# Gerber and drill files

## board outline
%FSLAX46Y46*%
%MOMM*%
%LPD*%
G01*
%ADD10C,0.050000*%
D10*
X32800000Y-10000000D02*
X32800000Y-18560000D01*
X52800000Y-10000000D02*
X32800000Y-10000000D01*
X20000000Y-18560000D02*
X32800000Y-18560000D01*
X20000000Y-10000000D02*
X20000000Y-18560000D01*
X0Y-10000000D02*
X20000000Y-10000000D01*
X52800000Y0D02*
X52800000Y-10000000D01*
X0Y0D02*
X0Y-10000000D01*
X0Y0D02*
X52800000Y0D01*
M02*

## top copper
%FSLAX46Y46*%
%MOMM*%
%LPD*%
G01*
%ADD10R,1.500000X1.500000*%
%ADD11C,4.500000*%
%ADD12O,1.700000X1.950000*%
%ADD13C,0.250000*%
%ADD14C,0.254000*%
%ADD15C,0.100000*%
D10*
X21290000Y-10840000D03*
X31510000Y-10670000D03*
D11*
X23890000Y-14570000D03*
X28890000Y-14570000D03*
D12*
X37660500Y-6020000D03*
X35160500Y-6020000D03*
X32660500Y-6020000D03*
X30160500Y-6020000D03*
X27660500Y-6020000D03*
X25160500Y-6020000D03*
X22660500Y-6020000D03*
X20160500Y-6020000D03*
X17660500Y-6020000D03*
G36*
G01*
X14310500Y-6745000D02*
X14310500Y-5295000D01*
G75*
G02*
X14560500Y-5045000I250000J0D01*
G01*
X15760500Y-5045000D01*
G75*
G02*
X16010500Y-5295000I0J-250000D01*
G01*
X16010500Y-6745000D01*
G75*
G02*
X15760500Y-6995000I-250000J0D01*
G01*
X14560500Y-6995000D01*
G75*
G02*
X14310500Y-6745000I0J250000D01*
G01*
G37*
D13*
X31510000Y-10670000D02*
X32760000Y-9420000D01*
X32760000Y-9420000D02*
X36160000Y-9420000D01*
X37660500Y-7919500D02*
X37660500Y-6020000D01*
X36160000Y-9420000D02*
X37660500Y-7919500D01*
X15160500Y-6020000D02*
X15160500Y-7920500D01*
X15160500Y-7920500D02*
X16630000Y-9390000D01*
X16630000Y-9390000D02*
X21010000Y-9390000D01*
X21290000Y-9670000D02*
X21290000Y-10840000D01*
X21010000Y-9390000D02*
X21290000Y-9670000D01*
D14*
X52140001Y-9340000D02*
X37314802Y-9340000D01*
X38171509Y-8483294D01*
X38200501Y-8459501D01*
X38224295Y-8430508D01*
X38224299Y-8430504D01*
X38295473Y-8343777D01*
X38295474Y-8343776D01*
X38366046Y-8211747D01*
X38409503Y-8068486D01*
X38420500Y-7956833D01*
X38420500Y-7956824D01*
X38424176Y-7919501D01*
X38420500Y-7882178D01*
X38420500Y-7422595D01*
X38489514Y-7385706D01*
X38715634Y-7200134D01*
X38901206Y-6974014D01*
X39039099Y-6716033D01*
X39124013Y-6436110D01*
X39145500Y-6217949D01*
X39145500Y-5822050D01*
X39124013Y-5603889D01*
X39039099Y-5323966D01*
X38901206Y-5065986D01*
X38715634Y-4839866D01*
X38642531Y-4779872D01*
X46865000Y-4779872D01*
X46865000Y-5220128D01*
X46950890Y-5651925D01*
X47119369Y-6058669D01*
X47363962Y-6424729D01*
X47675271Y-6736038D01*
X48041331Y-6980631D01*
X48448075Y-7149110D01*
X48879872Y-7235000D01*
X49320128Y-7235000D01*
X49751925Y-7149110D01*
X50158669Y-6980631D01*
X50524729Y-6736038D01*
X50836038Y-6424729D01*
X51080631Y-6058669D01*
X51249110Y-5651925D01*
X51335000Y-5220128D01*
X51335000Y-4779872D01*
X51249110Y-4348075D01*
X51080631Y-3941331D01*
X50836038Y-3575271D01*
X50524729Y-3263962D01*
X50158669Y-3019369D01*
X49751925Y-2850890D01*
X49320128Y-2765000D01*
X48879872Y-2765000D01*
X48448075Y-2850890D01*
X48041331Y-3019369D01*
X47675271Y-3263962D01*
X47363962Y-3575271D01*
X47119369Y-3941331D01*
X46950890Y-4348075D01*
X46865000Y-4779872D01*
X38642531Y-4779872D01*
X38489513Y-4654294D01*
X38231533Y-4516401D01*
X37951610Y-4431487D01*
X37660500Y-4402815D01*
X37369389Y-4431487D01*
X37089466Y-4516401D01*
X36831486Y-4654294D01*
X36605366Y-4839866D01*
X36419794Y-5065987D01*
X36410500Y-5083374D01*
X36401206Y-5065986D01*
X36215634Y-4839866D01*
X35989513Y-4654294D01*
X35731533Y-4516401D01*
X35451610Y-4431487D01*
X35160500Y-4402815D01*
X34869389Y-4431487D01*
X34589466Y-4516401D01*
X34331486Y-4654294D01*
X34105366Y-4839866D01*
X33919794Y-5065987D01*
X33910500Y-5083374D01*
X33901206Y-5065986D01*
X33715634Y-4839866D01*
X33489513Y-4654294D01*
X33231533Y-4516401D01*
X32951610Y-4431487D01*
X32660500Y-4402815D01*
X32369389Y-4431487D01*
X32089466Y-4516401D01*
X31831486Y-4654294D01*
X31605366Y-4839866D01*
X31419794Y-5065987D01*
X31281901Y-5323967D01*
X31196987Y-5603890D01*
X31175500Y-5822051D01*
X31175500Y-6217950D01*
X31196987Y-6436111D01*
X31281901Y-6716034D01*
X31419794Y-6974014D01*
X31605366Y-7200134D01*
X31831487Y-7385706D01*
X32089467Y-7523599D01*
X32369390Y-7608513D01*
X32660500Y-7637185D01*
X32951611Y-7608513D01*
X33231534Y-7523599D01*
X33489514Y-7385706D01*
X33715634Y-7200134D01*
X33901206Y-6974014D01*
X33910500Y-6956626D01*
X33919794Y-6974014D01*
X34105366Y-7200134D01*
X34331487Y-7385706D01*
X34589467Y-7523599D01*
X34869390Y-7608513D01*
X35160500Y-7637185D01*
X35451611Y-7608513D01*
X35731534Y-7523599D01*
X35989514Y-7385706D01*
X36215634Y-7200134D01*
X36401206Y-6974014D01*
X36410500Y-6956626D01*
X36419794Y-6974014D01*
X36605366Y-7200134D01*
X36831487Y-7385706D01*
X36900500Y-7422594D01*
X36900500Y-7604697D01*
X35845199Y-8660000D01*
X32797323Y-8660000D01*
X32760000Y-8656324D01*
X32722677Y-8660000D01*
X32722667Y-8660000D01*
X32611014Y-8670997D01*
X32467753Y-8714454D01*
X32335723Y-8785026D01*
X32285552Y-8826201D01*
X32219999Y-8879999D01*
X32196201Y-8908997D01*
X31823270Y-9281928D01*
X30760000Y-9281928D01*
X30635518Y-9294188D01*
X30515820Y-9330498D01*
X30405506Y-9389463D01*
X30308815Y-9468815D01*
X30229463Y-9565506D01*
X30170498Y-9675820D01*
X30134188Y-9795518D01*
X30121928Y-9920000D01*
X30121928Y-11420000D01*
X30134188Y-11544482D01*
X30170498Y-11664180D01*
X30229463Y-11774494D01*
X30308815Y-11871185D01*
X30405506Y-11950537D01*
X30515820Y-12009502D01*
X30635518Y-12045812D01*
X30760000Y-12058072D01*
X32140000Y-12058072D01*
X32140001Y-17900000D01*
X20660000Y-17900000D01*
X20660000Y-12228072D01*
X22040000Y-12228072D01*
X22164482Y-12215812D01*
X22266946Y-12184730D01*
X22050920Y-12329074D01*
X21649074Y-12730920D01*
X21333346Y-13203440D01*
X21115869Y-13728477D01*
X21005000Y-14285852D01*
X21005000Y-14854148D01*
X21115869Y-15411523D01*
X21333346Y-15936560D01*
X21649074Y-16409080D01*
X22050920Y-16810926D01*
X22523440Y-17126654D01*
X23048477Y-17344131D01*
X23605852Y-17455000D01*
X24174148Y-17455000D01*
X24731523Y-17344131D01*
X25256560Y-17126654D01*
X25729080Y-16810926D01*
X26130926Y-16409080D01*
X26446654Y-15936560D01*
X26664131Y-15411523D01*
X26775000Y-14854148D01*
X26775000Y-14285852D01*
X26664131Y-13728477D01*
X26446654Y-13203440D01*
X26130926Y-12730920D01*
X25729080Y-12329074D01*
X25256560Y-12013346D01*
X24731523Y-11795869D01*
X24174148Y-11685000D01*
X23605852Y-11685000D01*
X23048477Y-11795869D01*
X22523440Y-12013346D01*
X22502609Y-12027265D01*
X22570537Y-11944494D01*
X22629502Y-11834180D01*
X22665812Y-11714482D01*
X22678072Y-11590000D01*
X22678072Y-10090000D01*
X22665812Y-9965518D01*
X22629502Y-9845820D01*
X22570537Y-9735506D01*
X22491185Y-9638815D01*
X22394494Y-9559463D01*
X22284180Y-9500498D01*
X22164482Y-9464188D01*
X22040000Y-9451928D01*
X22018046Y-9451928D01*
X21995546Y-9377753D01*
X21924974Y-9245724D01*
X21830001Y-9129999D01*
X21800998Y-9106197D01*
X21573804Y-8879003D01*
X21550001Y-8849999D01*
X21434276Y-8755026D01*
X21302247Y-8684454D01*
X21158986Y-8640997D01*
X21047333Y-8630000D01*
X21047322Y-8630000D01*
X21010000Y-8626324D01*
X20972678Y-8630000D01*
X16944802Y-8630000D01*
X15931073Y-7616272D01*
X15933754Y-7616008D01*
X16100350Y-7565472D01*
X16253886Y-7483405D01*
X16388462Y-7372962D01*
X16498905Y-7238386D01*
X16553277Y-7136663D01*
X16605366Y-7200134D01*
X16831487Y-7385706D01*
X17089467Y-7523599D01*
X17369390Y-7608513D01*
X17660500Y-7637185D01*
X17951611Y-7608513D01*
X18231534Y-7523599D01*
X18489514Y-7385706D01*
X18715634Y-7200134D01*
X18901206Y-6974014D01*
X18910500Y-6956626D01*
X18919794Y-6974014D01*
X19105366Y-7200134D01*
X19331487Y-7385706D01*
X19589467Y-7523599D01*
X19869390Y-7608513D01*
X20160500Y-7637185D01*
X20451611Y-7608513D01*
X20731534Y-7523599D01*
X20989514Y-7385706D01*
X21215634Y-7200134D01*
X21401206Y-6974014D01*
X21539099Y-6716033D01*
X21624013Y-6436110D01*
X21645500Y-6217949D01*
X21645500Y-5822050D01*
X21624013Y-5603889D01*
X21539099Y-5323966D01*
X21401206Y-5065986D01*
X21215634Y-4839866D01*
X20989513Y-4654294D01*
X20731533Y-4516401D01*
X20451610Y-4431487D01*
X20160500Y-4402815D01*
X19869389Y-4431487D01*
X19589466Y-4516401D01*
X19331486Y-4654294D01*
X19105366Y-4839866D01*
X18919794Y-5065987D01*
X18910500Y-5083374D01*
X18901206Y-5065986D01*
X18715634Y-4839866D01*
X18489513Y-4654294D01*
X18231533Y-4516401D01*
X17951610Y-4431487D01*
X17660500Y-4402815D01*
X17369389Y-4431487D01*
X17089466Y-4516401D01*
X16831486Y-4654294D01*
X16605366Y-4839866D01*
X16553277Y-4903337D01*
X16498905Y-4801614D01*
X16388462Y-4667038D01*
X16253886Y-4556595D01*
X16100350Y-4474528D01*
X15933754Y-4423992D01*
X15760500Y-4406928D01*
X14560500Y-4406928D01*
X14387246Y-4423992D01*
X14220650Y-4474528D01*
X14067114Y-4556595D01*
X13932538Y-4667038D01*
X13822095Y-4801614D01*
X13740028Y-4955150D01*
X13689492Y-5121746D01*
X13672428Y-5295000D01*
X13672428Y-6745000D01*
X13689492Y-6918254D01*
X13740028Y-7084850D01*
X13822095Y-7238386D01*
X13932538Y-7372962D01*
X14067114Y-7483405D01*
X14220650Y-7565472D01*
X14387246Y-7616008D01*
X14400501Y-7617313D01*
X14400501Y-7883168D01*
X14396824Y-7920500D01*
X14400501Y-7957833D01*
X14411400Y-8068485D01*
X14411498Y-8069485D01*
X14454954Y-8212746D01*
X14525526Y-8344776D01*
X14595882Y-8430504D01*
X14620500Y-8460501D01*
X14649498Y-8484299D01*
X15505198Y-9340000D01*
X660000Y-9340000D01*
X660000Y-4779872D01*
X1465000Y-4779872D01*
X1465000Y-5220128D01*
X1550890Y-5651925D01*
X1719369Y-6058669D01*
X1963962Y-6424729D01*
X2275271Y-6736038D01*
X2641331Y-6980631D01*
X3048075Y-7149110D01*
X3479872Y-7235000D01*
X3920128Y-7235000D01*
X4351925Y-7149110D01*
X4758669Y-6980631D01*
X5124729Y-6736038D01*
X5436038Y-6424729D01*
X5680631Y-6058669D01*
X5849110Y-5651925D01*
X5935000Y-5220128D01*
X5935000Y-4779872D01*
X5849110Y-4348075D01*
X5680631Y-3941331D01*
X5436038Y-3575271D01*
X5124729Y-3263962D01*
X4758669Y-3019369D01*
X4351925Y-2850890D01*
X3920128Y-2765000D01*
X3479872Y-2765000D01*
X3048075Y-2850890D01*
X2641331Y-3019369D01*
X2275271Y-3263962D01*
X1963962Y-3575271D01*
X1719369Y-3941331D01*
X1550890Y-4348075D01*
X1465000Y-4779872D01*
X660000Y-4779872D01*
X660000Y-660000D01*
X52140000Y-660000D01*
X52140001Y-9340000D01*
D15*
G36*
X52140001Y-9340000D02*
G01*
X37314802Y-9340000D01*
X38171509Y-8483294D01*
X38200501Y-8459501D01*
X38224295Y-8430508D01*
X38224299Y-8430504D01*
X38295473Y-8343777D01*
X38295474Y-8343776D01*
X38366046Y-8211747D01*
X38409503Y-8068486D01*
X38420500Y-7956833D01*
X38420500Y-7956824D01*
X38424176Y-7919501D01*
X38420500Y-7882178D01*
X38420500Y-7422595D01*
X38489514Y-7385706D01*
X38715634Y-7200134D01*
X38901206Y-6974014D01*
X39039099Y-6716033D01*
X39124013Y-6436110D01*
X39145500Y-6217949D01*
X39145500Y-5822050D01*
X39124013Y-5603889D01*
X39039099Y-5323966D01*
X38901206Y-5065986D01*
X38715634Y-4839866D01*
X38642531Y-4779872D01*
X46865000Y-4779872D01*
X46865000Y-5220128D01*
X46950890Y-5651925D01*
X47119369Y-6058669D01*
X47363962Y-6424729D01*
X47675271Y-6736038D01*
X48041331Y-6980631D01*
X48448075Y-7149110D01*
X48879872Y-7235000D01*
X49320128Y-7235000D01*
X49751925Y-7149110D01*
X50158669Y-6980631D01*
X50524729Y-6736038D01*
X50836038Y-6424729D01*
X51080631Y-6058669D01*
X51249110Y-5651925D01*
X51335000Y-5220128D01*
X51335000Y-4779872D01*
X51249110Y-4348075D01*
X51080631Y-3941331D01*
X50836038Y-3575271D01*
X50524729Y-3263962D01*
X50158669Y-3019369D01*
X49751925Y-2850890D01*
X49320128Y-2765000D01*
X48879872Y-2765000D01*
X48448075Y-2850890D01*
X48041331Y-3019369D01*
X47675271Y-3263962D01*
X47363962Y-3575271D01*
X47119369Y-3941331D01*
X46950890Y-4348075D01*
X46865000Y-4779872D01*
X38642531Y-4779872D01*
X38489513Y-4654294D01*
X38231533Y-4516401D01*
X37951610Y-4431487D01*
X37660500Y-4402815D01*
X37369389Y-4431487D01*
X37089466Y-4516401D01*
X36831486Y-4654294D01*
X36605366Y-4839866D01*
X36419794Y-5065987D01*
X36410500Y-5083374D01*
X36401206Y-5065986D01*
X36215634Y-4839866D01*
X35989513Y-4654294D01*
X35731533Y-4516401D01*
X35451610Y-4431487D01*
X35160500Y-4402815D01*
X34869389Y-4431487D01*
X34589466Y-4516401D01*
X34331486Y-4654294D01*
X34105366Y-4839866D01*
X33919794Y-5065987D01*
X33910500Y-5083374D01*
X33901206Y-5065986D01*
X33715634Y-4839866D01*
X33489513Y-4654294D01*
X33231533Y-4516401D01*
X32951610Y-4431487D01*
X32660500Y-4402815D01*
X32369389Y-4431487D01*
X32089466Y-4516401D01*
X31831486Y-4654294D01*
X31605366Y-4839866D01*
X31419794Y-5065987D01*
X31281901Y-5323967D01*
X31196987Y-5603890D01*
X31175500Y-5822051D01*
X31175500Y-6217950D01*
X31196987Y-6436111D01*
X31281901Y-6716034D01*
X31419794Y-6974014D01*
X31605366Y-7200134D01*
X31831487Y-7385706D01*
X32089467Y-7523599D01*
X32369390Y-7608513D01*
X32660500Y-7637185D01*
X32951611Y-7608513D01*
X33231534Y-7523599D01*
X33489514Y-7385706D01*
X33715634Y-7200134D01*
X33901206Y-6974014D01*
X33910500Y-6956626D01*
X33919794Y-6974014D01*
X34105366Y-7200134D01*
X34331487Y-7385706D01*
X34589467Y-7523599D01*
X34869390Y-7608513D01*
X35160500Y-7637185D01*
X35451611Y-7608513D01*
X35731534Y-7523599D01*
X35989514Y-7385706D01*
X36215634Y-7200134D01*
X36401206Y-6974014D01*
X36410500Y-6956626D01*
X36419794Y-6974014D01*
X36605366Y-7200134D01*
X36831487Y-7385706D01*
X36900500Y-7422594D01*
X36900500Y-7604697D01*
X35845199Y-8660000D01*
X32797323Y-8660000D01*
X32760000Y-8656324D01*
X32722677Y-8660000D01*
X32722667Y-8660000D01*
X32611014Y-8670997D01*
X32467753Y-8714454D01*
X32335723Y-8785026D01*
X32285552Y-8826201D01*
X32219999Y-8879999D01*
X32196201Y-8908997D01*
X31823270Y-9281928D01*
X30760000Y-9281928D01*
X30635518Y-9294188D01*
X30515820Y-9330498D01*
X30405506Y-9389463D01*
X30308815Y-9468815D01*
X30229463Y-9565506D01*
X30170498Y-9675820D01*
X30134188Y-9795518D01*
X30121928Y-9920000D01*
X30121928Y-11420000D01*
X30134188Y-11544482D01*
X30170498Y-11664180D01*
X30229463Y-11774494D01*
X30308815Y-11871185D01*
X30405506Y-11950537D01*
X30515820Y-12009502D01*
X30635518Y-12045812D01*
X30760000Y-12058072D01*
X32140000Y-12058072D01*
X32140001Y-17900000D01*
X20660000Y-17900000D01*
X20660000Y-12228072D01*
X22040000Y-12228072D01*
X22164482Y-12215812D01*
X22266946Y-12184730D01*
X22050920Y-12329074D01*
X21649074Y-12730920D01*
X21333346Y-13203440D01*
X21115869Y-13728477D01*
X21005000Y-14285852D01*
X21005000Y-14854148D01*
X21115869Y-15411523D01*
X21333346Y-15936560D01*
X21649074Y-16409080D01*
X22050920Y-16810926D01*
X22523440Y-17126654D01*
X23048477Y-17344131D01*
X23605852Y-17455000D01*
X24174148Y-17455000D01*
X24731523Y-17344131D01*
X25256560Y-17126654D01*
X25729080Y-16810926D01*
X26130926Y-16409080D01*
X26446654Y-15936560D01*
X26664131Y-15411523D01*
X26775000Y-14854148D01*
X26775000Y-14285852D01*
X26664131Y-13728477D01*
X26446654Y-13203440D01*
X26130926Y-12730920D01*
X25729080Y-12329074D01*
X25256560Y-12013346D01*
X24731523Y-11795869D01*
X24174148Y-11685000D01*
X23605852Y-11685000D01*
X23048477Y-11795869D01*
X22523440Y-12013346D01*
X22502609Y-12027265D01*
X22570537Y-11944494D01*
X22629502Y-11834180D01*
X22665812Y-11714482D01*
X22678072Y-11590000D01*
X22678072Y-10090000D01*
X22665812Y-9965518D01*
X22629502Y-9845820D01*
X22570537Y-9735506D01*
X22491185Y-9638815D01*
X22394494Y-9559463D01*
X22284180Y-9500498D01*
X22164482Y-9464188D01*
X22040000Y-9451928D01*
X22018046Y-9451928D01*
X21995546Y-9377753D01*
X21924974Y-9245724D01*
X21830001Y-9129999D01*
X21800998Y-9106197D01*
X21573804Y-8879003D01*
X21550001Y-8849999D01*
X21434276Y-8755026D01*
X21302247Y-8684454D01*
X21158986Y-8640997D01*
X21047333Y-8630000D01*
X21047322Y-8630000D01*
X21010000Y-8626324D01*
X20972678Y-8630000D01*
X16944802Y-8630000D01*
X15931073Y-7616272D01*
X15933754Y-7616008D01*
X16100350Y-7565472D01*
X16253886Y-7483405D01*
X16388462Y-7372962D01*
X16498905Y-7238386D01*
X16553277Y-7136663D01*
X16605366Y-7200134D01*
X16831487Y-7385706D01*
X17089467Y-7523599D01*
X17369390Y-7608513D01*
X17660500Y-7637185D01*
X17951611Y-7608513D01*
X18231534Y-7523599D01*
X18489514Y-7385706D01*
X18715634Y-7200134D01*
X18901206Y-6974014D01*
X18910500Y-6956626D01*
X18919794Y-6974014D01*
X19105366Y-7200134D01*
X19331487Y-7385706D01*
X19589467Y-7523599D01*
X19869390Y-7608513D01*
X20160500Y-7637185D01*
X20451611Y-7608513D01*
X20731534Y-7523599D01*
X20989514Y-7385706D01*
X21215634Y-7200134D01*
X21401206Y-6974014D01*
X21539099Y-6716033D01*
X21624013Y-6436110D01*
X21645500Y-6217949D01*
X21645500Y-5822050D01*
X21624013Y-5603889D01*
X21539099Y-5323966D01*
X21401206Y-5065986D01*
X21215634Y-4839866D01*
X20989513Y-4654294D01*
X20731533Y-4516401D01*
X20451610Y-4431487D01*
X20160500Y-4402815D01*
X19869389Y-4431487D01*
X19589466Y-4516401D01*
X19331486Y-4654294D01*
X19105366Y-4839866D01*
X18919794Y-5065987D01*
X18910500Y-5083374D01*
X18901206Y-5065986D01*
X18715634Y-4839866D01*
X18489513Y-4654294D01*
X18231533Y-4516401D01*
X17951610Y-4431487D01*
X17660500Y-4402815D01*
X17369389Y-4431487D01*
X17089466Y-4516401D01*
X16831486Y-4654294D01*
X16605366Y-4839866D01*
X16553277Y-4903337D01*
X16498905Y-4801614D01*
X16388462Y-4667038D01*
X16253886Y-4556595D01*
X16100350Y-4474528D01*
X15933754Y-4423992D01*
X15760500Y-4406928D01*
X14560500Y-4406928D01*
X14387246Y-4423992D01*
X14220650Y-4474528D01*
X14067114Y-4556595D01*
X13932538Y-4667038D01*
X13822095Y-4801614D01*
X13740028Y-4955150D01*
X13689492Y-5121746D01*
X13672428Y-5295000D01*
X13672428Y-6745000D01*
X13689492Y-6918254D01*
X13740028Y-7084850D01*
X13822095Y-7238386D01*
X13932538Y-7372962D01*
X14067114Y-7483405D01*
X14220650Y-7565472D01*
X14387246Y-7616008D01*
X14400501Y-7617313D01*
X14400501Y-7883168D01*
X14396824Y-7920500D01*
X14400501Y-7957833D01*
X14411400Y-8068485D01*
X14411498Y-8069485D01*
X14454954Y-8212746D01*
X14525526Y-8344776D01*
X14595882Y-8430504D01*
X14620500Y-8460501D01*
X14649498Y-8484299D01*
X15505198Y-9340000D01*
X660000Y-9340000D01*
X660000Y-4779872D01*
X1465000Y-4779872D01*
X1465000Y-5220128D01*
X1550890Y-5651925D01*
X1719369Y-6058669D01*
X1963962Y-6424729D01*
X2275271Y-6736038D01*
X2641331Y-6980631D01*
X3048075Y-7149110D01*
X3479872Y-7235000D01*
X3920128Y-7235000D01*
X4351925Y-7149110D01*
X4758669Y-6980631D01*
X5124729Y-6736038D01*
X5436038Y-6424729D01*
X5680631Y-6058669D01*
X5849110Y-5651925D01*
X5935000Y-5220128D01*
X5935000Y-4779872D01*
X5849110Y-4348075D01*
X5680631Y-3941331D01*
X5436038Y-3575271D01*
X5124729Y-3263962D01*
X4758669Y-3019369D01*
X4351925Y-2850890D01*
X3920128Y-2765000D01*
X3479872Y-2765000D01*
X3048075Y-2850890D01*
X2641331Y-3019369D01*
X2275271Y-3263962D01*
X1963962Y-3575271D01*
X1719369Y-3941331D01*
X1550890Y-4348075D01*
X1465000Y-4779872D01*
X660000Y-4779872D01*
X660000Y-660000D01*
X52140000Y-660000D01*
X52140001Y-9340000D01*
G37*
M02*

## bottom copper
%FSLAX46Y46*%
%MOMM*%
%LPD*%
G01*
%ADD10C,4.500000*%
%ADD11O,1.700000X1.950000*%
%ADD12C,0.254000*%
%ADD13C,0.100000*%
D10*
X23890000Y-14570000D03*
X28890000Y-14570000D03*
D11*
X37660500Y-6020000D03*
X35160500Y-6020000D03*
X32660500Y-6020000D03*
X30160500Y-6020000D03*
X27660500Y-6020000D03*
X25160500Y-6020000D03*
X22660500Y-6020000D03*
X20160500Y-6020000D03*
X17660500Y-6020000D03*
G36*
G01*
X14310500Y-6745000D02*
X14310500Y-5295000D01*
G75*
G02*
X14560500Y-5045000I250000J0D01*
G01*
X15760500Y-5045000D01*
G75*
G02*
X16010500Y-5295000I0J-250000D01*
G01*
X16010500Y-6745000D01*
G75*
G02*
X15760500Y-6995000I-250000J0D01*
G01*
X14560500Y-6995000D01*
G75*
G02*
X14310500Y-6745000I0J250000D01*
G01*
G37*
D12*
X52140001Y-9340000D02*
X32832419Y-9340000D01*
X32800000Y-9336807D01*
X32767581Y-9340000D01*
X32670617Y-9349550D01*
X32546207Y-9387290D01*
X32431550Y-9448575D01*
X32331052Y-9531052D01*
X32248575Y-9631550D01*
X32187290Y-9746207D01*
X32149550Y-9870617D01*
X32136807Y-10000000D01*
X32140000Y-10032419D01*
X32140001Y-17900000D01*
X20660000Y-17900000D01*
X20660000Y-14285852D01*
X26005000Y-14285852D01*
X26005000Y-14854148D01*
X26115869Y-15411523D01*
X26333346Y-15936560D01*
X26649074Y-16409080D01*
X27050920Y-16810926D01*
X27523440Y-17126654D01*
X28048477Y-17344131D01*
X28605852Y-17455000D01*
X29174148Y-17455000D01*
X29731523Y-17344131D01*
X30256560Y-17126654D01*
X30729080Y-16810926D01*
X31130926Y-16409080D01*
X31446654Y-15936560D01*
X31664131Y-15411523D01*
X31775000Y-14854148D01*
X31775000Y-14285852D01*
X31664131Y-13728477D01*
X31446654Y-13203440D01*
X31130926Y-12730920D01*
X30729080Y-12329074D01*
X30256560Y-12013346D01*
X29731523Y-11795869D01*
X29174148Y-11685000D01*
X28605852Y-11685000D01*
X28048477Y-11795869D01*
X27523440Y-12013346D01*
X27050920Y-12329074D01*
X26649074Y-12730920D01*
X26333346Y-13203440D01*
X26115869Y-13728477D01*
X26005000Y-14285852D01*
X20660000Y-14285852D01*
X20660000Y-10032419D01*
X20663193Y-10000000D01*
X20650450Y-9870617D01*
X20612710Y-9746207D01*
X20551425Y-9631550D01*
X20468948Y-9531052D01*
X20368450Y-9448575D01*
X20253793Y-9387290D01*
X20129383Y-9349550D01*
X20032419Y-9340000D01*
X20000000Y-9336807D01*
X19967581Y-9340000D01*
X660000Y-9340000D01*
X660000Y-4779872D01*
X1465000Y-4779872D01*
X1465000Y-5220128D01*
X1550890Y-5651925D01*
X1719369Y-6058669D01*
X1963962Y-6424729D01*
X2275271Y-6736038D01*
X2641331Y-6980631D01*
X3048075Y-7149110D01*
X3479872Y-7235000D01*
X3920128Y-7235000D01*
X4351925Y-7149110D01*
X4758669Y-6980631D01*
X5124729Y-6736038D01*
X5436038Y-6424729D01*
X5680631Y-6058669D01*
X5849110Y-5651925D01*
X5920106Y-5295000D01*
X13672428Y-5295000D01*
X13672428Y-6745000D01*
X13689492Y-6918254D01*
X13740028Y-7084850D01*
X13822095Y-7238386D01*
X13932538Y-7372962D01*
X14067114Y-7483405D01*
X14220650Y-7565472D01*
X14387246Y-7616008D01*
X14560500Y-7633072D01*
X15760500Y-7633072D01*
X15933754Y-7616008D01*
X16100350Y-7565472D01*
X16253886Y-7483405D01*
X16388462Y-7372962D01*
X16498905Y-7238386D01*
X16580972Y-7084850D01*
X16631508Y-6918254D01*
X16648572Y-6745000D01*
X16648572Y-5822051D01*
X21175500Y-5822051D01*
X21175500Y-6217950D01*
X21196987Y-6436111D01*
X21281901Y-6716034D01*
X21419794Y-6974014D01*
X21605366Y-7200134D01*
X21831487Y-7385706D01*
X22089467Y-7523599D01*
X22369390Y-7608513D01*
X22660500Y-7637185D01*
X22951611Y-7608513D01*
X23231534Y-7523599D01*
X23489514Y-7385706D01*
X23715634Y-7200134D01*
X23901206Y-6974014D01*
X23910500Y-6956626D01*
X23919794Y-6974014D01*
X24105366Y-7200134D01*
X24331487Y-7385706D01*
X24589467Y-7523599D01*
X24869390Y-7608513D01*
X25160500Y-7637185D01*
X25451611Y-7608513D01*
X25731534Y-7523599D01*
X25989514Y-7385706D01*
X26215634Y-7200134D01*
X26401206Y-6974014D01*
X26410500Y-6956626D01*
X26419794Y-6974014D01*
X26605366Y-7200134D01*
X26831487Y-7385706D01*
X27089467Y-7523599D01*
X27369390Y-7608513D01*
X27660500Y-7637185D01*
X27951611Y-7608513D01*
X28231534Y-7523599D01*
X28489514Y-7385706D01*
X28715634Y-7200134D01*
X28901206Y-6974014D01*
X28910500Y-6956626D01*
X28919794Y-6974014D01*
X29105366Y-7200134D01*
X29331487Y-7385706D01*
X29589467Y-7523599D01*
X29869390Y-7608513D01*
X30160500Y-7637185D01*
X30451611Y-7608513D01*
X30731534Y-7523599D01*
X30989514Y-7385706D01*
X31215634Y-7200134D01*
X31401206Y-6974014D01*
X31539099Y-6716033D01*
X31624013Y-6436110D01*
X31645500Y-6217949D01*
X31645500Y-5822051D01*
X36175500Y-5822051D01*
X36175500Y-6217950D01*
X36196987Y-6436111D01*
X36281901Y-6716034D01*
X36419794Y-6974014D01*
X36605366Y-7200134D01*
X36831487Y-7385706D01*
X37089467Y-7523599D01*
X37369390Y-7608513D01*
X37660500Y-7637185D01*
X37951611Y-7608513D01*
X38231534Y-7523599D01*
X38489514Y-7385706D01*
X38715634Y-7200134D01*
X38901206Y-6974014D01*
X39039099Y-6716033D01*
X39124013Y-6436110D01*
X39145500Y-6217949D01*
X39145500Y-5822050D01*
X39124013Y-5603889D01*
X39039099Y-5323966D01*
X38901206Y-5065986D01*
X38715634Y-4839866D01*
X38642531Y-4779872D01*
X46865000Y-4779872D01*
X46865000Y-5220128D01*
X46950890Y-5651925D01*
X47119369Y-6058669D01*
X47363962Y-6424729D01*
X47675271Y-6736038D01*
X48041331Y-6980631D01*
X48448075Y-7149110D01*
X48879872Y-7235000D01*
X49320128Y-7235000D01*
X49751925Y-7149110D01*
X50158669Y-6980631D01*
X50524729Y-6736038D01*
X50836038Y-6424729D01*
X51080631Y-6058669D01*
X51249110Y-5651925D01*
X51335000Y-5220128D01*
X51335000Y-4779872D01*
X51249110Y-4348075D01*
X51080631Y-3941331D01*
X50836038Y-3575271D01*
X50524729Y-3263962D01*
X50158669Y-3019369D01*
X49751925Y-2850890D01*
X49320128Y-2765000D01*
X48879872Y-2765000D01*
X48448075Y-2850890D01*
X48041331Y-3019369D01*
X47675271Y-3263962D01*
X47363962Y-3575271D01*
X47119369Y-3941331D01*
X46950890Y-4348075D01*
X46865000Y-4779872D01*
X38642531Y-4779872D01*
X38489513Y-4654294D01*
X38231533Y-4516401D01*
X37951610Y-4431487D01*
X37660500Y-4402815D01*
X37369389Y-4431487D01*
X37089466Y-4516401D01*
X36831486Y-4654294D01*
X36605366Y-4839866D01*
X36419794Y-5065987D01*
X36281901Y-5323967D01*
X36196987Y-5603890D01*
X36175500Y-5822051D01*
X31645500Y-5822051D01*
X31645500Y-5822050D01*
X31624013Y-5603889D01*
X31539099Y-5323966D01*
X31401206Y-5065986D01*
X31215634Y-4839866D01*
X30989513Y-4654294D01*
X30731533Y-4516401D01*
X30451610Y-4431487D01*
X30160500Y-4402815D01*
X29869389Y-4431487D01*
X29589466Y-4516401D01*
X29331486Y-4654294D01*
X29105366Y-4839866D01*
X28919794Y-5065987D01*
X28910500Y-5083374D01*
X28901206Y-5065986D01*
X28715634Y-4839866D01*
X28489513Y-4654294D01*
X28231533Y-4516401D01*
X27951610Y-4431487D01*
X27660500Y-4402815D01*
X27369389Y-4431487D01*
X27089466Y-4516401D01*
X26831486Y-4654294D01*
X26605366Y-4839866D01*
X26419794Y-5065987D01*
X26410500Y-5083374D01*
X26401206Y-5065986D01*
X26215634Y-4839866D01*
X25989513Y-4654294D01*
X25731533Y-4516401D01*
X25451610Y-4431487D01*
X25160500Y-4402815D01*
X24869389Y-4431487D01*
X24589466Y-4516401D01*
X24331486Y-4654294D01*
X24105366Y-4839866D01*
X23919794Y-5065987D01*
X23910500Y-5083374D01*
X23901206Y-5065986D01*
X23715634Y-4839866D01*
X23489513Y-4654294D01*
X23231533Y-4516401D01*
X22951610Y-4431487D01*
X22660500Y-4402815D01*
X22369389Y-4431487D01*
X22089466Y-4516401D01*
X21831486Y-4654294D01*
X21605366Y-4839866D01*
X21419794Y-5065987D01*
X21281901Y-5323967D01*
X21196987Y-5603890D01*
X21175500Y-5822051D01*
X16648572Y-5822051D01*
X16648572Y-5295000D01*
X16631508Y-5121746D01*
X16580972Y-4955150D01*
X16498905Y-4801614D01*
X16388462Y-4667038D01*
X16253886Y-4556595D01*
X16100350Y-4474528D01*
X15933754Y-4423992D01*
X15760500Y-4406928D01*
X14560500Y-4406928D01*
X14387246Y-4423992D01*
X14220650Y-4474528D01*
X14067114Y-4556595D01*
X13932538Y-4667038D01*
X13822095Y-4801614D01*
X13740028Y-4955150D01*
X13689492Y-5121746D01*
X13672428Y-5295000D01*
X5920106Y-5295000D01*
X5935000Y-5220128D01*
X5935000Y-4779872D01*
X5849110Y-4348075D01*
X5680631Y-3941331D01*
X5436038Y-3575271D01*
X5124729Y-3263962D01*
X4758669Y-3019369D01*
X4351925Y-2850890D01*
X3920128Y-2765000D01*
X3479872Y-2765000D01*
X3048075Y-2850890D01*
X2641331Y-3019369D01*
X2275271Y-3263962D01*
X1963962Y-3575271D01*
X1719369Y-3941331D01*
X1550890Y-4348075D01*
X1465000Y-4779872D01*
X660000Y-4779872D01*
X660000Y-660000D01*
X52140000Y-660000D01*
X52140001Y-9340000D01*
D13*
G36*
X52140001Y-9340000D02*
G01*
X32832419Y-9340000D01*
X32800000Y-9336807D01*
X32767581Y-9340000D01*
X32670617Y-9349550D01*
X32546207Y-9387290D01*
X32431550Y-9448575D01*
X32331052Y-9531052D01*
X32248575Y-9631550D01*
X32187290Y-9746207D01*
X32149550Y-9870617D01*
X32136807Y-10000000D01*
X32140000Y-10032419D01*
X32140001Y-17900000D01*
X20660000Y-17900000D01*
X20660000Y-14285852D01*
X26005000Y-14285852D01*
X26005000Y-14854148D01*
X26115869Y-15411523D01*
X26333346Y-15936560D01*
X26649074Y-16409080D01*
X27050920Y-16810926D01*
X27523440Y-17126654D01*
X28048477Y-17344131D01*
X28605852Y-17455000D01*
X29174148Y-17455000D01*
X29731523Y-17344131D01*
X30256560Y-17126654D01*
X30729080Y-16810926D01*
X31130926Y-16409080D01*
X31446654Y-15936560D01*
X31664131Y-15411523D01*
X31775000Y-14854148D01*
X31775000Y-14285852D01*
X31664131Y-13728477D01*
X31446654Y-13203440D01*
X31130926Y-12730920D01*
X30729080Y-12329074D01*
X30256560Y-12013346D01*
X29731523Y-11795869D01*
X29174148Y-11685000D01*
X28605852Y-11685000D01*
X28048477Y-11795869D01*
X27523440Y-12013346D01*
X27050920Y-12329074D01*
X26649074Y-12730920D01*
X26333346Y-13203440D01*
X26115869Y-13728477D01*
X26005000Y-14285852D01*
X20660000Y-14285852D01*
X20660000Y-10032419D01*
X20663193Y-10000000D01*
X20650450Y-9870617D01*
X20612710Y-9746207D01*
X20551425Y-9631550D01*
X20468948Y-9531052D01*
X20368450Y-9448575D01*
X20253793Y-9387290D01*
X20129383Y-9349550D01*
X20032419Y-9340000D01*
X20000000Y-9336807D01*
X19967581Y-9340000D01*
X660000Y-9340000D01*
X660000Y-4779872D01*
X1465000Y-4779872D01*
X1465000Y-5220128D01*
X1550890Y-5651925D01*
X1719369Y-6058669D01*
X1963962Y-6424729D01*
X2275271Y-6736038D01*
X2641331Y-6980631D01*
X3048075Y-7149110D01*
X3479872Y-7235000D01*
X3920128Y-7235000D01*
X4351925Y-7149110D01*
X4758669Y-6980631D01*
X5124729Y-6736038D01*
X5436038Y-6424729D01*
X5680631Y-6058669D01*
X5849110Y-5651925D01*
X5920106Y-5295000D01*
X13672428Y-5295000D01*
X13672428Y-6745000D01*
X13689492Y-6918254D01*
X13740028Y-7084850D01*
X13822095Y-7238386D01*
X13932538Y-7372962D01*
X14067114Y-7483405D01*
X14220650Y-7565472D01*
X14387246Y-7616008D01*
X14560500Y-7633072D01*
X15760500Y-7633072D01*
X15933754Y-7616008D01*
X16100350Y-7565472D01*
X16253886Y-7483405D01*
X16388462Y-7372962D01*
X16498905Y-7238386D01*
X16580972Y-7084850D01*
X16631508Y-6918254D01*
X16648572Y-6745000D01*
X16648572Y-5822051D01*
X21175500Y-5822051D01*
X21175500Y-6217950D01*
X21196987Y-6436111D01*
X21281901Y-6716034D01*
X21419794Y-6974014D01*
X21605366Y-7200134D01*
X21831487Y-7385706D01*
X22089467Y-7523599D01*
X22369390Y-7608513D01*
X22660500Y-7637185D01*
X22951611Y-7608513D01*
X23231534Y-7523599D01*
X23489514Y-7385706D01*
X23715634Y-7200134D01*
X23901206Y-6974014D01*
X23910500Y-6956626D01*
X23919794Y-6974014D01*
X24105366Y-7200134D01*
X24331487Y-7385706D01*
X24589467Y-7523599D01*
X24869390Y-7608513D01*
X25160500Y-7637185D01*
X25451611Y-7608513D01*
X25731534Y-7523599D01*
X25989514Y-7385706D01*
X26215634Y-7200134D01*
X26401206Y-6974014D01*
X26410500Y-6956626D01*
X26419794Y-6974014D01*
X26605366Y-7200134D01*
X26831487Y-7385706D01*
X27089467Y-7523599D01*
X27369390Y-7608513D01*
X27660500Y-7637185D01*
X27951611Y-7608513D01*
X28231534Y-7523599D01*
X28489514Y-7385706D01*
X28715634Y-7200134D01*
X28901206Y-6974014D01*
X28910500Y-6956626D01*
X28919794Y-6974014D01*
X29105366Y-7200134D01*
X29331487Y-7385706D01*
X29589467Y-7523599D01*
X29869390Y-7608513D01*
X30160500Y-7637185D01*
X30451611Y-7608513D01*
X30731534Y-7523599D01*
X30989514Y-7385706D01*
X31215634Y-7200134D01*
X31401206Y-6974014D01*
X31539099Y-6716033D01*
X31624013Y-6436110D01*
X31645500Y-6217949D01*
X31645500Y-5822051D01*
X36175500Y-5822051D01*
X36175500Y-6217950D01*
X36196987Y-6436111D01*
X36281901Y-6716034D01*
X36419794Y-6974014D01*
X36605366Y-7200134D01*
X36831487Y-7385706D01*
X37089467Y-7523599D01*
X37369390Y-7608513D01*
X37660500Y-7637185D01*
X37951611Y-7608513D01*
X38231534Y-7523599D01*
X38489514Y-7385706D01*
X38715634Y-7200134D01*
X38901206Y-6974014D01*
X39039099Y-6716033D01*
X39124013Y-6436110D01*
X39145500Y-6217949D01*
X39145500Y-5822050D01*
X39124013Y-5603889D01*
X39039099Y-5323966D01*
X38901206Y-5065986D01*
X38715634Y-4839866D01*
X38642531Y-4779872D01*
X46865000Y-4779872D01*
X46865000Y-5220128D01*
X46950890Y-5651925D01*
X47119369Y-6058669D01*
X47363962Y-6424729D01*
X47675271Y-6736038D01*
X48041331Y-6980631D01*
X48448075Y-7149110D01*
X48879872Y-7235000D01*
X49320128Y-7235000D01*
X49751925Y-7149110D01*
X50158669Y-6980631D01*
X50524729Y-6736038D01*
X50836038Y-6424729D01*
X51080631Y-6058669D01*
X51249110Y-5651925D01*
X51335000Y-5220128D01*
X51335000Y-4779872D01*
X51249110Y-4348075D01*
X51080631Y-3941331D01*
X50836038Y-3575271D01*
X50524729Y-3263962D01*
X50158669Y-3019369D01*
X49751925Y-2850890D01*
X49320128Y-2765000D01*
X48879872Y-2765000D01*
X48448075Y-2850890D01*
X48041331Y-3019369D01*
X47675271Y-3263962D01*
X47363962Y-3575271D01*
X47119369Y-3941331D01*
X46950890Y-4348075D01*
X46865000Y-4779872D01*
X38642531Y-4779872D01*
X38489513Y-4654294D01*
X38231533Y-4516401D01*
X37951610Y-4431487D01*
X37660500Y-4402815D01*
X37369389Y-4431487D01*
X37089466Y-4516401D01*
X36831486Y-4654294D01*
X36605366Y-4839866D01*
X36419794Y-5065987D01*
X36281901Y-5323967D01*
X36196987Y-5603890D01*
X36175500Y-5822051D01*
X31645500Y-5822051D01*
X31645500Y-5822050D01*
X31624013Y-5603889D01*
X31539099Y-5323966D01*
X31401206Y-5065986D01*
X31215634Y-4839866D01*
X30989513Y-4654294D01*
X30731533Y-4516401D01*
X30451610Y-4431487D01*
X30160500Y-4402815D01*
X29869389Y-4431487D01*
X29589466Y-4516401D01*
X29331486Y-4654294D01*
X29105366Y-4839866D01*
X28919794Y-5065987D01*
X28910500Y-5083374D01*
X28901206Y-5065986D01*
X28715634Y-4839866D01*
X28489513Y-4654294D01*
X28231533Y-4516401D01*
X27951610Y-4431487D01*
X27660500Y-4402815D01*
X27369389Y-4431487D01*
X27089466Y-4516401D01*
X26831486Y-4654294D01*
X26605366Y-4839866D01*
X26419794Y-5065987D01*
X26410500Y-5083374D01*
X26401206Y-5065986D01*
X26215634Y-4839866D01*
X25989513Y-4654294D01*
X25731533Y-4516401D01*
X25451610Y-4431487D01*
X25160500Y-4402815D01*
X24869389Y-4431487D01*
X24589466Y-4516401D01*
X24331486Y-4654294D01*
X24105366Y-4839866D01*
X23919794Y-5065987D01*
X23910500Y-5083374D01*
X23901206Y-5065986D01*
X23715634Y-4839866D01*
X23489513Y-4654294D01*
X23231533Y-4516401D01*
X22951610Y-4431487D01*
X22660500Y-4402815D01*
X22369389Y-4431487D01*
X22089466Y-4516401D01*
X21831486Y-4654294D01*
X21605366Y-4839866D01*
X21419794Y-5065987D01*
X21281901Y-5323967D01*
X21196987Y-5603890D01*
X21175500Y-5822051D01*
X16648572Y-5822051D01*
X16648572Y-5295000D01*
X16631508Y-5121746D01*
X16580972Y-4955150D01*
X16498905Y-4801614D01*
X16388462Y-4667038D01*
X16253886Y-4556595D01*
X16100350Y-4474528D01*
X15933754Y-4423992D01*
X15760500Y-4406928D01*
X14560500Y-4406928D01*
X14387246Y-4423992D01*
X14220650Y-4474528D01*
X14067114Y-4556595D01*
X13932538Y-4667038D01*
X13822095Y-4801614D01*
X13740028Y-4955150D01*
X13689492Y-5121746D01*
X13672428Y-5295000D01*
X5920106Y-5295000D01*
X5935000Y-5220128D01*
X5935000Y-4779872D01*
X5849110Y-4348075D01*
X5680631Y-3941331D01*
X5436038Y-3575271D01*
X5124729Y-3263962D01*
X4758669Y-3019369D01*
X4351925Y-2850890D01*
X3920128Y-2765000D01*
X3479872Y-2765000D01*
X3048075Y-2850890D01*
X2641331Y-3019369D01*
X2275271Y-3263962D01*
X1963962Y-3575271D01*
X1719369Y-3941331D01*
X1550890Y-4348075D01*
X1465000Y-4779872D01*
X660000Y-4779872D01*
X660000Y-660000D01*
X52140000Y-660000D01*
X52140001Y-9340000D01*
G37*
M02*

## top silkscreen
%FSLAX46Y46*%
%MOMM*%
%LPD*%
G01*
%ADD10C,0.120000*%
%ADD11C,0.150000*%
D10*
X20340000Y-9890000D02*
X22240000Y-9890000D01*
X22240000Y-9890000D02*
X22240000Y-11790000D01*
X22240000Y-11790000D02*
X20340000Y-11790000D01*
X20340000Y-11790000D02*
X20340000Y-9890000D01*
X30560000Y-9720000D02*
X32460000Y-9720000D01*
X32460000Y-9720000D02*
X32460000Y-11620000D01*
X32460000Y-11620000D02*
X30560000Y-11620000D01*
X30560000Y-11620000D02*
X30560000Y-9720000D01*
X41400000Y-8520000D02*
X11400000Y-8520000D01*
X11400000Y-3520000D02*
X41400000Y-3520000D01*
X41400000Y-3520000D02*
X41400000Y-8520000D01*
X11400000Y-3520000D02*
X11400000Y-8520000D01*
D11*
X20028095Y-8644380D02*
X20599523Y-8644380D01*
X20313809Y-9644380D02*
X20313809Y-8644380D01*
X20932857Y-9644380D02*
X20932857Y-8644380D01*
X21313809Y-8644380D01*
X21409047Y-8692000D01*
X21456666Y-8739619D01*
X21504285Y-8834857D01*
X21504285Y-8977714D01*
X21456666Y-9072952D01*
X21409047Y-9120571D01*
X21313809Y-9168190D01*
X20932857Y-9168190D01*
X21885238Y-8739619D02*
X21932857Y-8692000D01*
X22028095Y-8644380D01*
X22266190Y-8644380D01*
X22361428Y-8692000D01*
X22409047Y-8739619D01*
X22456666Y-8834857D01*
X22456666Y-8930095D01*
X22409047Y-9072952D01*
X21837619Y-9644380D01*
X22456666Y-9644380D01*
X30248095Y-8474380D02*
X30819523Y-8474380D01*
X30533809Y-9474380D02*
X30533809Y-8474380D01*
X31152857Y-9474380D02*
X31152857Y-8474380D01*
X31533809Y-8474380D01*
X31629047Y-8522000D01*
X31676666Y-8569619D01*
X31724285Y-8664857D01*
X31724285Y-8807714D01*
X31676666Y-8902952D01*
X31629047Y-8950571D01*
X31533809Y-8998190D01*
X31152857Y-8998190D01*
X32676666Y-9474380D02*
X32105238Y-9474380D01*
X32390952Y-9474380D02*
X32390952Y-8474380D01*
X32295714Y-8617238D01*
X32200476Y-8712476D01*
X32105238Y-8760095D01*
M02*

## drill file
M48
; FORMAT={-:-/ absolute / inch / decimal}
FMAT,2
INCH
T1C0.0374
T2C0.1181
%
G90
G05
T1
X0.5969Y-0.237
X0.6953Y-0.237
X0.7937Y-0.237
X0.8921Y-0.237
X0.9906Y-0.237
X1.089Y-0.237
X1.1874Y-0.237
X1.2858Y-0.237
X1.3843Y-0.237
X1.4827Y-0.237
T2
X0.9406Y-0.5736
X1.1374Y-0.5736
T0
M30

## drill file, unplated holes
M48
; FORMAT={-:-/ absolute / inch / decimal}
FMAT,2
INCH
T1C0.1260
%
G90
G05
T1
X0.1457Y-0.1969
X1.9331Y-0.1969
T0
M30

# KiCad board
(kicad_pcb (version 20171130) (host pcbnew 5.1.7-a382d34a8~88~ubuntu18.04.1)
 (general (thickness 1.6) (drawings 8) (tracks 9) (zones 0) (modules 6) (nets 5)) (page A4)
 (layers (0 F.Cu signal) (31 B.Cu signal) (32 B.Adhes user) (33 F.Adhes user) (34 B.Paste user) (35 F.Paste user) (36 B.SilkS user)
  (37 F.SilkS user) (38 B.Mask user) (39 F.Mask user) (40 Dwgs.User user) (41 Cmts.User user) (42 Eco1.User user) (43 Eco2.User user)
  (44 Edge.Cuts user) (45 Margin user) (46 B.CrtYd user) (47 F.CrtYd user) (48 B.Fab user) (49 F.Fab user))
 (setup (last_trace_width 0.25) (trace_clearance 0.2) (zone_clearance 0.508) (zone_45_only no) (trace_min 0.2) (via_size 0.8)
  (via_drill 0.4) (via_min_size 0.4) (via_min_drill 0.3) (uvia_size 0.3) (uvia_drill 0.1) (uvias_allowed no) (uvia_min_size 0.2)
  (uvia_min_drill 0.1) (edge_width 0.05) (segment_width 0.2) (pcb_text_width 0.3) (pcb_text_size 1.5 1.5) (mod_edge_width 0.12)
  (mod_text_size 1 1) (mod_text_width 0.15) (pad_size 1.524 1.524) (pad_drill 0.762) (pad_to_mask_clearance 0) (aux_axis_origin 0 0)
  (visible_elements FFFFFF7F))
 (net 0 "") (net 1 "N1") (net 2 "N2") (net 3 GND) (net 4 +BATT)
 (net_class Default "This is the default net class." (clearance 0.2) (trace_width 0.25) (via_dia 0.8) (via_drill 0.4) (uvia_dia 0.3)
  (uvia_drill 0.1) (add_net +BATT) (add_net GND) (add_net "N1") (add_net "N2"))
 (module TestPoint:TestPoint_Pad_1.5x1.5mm (layer F.Cu) (at 21.29 10.84)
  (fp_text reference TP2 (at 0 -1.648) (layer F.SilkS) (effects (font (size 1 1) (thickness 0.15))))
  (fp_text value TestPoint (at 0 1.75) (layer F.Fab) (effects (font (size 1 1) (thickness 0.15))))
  (fp_line (start -0.95 -0.95) (end 0.95 -0.95) (layer F.SilkS) (width 0.12))
  (fp_line (start 0.95 -0.95) (end 0.95 0.95) (layer F.SilkS) (width 0.12))
  (fp_line (start 0.95 0.95) (end -0.95 0.95) (layer F.SilkS) (width 0.12))
  (fp_line (start -0.95 0.95) (end -0.95 -0.95) (layer F.SilkS) (width 0.12))
  (pad 1 smd rect (at 0 0) (size 1.5 1.5) (layers F.Cu F.Mask) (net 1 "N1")))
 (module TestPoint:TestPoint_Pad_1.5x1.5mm (layer F.Cu) (at 31.51 10.67)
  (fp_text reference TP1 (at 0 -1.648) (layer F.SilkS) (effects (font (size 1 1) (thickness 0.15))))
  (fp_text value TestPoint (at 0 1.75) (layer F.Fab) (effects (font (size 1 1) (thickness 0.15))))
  (fp_line (start -0.95 -0.95) (end 0.95 -0.95) (layer F.SilkS) (width 0.12))
  (fp_line (start 0.95 -0.95) (end 0.95 0.95) (layer F.SilkS) (width 0.12))
  (fp_line (start 0.95 0.95) (end -0.95 0.95) (layer F.SilkS) (width 0.12))
  (fp_line (start -0.95 0.95) (end -0.95 -0.95) (layer F.SilkS) (width 0.12))
  (pad 1 smd rect (at 0 0) (size 1.5 1.5) (layers F.Cu F.Mask) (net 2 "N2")))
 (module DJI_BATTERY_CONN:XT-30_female (layer B.Cu) (at 26.39 14.57 180)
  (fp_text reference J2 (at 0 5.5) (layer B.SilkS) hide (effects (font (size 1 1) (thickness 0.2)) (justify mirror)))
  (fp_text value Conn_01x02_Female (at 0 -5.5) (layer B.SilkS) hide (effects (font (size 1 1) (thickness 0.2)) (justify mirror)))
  (pad 1 thru_hole circle (at 2.5 0 180) (size 4.5 4.5) (drill 3) (layers *.Cu *.Mask) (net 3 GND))
  (pad 2 thru_hole circle (at -2.5 0 180) (size 4.5 4.5) (drill 3) (layers *.Cu *.Mask) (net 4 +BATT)))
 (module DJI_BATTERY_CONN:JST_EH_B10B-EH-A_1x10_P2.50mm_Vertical (layer F.Cu) (at 26.4 6.02)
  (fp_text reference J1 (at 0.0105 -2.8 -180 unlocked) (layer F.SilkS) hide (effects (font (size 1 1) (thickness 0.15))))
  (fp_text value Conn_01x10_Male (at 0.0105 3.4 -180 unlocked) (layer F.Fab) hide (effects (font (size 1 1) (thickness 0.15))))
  (fp_line (start 15 2.5) (end -15 2.5) (layer F.SilkS) (width 0.12))
  (fp_line (start -15 -2.5) (end 15 -2.5) (layer F.SilkS) (width 0.12))
  (fp_line (start 15 -2.5) (end 15 2.5) (layer F.SilkS) (width 0.12))
  (fp_line (start -15 -2.5) (end -15 2.5) (layer F.SilkS) (width 0.12))
  (pad 10 thru_hole oval (at 11.2605 0) (size 1.7 1.95) (drill 0.95) (layers *.Cu *.Mask) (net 2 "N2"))
  (pad 9 thru_hole oval (at 8.7605 0) (size 1.7 1.95) (drill 0.95) (layers *.Cu *.Mask) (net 3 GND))
  (pad 8 thru_hole oval (at 6.2605 0) (size 1.7 1.95) (drill 0.95) (layers *.Cu *.Mask) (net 3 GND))
  (pad 7 thru_hole oval (at 3.7605 0) (size 1.7 1.95) (drill 0.95) (layers *.Cu *.Mask) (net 4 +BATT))
  (pad 6 thru_hole oval (at 1.2605 0) (size 1.7 1.95) (drill 0.95) (layers *.Cu *.Mask) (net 4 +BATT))
  (pad 5 thru_hole oval (at -1.2395 0) (size 1.7 1.95) (drill 0.95) (layers *.Cu *.Mask) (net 4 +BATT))
  (pad 4 thru_hole oval (at -3.7395 0) (size 1.7 1.95) (drill 0.95) (layers *.Cu *.Mask) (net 4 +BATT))
  (pad 3 thru_hole oval (at -6.2395 0) (size 1.7 1.95) (drill 0.95) (layers *.Cu *.Mask) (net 3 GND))
  (pad 2 thru_hole oval (at -8.7395 0) (size 1.7 1.95) (drill 0.95) (layers *.Cu *.Mask) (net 3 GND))
  (pad 1 thru_hole roundrect (at -11.2395 0) (size 1.7 1.95) (drill 0.95) (layers *.Cu *.Mask) (roundrect_rratio 0.1470588235294118)
   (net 1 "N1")))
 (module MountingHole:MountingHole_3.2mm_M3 (layer F.Cu) (at 3.7 5)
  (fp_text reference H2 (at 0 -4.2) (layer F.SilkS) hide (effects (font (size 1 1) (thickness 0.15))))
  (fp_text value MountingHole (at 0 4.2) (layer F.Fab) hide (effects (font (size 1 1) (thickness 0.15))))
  (pad 1 np_thru_hole circle (at 0 0) (size 3.2 3.2) (drill 3.2) (layers *.Cu *.Mask)))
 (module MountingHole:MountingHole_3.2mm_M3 (layer F.Cu) (at 49.1 5)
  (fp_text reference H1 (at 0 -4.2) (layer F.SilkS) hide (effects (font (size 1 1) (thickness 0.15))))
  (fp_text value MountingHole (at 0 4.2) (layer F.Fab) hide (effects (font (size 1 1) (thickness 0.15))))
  (pad 1 np_thru_hole circle (at 0 0) (size 3.2 3.2) (drill 3.2) (layers *.Cu *.Mask)))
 (gr_line (start 32.8 10) (end 32.8 18.56) (layer Edge.Cuts) (width 0.05))
 (gr_line (start 52.8 10) (end 32.8 10) (layer Edge.Cuts) (width 0.05))
 (gr_line (start 20 18.56) (end 32.8 18.56) (layer Edge.Cuts) (width 0.05))
 (gr_line (start 20 10) (end 20 18.56) (layer Edge.Cuts) (width 0.05))
 (gr_line (start 0 10) (end 20 10) (layer Edge.Cuts) (width 0.05))
 (gr_line (start 52.8 0) (end 52.8 10) (layer Edge.Cuts) (width 0.05))
 (gr_line (start 0 0) (end 0 10) (layer Edge.Cuts) (width 0.05))
 (gr_line (start 0 0) (end 52.8 0) (layer Edge.Cuts) (width 0.05))
 (segment (start 31.51 10.67) (end 32.76 9.42) (width 0.25) (layer F.Cu) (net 2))
 (segment (start 32.76 9.42) (end 36.16 9.42) (width 0.25) (layer F.Cu) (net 2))
 (segment (start 37.6605 7.9195) (end 37.6605 6.02) (width 0.25) (layer F.Cu) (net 2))
 (segment (start 36.16 9.42) (end 37.6605 7.9195) (width 0.25) (layer F.Cu) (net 2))
 (segment (start 15.1605 6.02) (end 15.1605 7.9205) (width 0.25) (layer F.Cu) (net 1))
 (segment (start 15.1605 7.9205) (end 16.63 9.39) (width 0.25) (layer F.Cu) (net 1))
 (segment (start 16.63 9.39) (end 21.01 9.39) (width 0.25) (layer F.Cu) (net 1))
 (segment (start 21.29 9.67) (end 21.29 10.84) (width 0.25) (layer F.Cu) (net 1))
 (segment (start 21.01 9.39) (end 21.29 9.67) (width 0.25) (layer F.Cu) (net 1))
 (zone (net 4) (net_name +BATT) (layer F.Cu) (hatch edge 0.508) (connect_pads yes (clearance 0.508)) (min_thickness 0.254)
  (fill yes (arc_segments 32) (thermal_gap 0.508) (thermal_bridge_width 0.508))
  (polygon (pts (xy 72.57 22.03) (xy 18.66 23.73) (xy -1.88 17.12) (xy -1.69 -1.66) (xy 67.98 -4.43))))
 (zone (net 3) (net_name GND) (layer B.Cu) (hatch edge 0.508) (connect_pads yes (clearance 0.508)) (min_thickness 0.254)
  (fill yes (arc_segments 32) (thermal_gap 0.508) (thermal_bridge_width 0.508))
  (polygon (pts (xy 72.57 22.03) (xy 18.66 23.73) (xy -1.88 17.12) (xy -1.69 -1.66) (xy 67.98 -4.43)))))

